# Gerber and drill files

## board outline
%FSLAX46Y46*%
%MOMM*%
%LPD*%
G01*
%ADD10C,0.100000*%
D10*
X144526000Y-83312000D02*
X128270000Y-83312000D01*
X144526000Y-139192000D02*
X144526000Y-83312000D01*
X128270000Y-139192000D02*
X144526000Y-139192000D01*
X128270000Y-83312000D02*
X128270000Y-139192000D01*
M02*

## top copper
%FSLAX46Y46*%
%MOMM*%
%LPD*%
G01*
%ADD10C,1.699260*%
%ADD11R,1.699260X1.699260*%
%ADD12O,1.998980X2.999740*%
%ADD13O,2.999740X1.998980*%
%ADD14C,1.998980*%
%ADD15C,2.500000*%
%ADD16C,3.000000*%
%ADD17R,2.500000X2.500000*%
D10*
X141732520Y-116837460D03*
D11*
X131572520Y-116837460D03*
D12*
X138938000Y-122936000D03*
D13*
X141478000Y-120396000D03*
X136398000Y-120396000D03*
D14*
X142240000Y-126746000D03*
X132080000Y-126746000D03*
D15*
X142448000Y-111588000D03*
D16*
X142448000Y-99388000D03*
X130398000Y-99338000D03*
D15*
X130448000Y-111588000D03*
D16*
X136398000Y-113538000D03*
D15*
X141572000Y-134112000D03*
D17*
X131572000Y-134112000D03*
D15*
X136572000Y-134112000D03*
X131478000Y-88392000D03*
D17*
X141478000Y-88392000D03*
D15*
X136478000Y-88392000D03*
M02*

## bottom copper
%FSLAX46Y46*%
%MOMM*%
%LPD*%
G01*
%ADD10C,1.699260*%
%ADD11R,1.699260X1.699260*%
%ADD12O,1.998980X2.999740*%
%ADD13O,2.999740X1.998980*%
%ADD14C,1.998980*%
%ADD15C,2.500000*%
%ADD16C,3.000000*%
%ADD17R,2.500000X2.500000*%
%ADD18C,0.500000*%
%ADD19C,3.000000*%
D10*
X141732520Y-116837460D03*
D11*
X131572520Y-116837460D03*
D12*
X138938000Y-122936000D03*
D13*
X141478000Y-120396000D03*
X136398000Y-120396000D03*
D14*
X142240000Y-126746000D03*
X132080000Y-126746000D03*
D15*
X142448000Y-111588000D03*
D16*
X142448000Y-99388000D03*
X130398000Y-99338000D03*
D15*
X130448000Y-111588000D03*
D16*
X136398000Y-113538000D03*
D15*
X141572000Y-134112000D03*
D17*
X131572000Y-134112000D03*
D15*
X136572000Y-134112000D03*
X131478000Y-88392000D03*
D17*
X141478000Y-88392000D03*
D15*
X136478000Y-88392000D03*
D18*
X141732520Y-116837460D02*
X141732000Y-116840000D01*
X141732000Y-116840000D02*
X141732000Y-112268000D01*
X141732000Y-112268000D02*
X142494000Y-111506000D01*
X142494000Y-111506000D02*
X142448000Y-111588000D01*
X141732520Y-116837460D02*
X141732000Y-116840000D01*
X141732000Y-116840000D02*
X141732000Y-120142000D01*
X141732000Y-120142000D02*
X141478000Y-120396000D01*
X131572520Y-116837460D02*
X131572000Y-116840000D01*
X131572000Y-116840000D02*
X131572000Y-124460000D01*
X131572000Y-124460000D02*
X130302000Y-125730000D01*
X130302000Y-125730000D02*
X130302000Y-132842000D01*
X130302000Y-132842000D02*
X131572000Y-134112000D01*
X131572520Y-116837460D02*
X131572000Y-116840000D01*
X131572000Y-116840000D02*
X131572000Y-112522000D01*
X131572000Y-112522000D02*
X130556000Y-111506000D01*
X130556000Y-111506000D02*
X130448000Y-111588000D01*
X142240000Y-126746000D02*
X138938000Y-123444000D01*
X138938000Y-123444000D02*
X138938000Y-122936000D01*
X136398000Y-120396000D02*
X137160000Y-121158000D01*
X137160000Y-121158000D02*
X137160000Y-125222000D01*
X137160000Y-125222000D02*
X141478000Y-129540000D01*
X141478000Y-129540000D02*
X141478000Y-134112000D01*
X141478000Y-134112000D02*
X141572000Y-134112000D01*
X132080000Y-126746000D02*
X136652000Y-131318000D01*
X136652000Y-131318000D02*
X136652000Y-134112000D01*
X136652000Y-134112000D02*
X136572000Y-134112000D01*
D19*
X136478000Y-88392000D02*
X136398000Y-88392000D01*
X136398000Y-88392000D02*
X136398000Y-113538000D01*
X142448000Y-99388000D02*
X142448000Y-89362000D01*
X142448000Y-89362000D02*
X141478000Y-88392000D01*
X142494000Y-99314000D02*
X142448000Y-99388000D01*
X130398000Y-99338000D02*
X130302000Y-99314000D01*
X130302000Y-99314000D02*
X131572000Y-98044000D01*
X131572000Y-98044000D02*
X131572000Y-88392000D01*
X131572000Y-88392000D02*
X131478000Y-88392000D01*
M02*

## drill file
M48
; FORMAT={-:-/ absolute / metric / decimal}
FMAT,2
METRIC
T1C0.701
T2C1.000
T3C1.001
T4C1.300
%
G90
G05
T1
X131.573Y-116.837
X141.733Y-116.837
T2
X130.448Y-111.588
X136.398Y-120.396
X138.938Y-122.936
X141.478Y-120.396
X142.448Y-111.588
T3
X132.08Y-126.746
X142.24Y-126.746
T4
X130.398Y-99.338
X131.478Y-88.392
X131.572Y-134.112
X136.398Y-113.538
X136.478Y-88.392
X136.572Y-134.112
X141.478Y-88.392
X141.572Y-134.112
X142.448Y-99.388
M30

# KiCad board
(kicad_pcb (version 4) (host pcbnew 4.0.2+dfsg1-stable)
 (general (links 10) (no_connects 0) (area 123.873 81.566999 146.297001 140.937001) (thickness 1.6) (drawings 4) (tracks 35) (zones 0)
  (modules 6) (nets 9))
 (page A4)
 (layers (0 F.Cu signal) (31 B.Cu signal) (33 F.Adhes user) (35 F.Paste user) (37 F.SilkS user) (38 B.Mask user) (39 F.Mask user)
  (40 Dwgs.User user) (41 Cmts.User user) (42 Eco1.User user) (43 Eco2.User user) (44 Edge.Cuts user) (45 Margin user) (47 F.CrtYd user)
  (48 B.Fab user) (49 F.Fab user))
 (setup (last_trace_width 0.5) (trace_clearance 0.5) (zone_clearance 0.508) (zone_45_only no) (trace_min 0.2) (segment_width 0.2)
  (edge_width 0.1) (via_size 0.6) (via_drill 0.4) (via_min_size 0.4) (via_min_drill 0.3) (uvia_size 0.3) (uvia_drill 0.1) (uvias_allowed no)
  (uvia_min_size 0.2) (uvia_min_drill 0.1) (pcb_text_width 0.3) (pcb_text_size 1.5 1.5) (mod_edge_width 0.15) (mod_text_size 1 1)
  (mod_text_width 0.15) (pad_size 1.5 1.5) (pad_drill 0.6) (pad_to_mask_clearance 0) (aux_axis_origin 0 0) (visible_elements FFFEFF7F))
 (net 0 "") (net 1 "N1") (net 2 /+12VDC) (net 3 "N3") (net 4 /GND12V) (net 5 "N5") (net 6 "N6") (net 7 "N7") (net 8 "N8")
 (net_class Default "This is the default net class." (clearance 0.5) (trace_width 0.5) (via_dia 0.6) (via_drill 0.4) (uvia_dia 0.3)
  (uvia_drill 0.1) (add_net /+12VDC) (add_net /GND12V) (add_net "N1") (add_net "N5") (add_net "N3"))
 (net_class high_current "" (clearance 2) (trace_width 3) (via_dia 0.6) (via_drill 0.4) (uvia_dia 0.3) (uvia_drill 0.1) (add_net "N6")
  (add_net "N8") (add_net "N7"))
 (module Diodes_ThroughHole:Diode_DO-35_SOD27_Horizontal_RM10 (layer F.Cu) (at 131.572 116.84)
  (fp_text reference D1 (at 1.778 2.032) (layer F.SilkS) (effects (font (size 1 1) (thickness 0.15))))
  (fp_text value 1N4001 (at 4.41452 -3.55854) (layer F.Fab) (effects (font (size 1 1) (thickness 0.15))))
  (pad 2 thru_hole circle (at 10.16052 -0.00254 180) (size 1.69926 1.69926) (drill 0.70104) (layers *.Cu *.Mask F.SilkS) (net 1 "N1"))
  (pad 1 thru_hole rect (at 0.00052 -0.00254 180) (size 1.69926 1.69926) (drill 0.70104) (layers *.Cu *.Mask F.SilkS) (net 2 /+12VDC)))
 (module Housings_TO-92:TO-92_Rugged (layer F.Cu) (at 141.478 120.396 180)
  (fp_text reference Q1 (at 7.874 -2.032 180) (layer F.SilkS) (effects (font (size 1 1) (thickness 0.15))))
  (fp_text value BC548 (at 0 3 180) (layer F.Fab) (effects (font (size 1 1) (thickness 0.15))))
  (pad 2 thru_hole oval (at 2.54 -2.54 270) (size 2.99974 1.99898) (drill 1) (layers *.Cu *.Mask F.SilkS) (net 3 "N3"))
  (pad 1 thru_hole oval (at 0 0 270) (size 1.99898 2.99974) (drill 1) (layers *.Cu *.Mask F.SilkS) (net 1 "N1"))
  (pad 3 thru_hole oval (at 5.08 0 270) (size 1.99898 2.99974) (drill 1) (layers *.Cu *.Mask F.SilkS) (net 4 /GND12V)))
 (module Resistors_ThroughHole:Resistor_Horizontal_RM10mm (layer F.Cu) (at 137.16 126.746 180)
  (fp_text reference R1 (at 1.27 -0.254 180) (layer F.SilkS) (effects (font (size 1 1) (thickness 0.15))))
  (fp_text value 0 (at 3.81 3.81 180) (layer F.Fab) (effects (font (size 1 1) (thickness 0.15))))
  (pad 1 thru_hole circle (at -5.08 0 180) (size 1.99898 1.99898) (drill 1.00076) (layers *.Cu *.SilkS *.Mask) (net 3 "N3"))
  (pad 2 thru_hole circle (at 5.08 0 180) (size 1.99898 1.99898) (drill 1.00076) (layers *.Cu *.SilkS *.Mask) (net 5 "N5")))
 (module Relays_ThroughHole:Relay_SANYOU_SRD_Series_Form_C (layer F.Cu) (at 136.398 113.538 90)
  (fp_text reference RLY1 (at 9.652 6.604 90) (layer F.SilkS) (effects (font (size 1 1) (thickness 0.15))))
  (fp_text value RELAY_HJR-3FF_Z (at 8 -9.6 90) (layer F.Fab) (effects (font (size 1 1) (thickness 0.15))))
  (pad 2 thru_hole circle (at 1.95 6.05 180) (size 2.5 2.5) (drill 1) (layers *.Cu *.Mask) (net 1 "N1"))
  (pad 3 thru_hole circle (at 14.15 6.05 180) (size 3 3) (drill 1.3) (layers *.Cu *.Mask) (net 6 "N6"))
  (pad 4 thru_hole circle (at 14.2 -6 180) (size 3 3) (drill 1.3) (layers *.Cu *.Mask) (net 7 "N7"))
  (pad 5 thru_hole circle (at 1.95 -5.95 180) (size 2.5 2.5) (drill 1) (layers *.Cu *.Mask F.SilkS) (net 2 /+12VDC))
  (pad 1 thru_hole circle (at 0 0 180) (size 3 3) (drill 1.3) (layers *.Cu *.Mask) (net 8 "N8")))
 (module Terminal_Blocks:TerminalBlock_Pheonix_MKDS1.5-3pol (layer F.Cu) (at 131.572 134.112)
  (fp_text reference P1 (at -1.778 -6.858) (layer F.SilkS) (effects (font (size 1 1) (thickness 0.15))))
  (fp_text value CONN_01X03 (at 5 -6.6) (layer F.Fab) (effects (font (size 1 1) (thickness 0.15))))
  (pad 3 thru_hole circle (at 10 0) (size 2.5 2.5) (drill 1.3) (layers *.Cu *.Mask F.SilkS) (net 4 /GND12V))
  (pad 1 thru_hole rect (at 0 0) (size 2.5 2.5) (drill 1.3) (layers *.Cu *.Mask F.SilkS) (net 2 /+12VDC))
  (pad 2 thru_hole circle (at 5 0) (size 2.5 2.5) (drill 1.3) (layers *.Cu *.Mask F.SilkS) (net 5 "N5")))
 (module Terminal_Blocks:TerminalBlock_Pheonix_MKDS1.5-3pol (layer F.Cu) (at 141.478 88.392 180)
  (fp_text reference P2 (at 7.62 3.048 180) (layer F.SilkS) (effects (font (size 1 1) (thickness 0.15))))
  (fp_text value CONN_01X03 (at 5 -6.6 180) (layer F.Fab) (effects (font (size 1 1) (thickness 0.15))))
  (pad 3 thru_hole circle (at 10 0 180) (size 2.5 2.5) (drill 1.3) (layers *.Cu *.Mask F.SilkS) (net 7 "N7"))
  (pad 1 thru_hole rect (at 0 0 180) (size 2.5 2.5) (drill 1.3) (layers *.Cu *.Mask F.SilkS) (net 6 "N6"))
  (pad 2 thru_hole circle (at 5 0 180) (size 2.5 2.5) (drill 1.3) (layers *.Cu *.Mask F.SilkS) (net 8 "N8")))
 (gr_line (start 144.526 83.312) (end 128.27 83.312) (angle 90) (layer Edge.Cuts) (width 0.1))
 (gr_line (start 144.526 139.192) (end 144.526 83.312) (angle 90) (layer Edge.Cuts) (width 0.1))
 (gr_line (start 128.27 139.192) (end 144.526 139.192) (angle 90) (layer Edge.Cuts) (width 0.1))
 (gr_line (start 128.27 83.312) (end 128.27 139.192) (angle 90) (layer Edge.Cuts) (width 0.1))
 (segment (start 141.73252 116.83746) (end 141.732 116.84) (width 0.5) (layer B.Cu) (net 1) (status 80000))
 (segment (start 141.732 116.84) (end 141.732 112.268) (width 0.5) (layer B.Cu) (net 1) (status 80000))
 (segment (start 141.732 112.268) (end 142.494 111.506) (width 0.5) (layer B.Cu) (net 1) (status 80000))
 (segment (start 142.494 111.506) (end 142.448 111.588) (width 0.5) (layer B.Cu) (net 1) (status 80000))
 (segment (start 141.73252 116.83746) (end 141.732 116.84) (width 0.5) (layer B.Cu) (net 1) (status 80000))
 (segment (start 141.732 116.84) (end 141.732 120.142) (width 0.5) (layer B.Cu) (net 1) (status 80000))
 (segment (start 141.732 120.142) (end 141.478 120.396) (width 0.5) (layer B.Cu) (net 1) (status 80000))
 (segment (start 131.57252 116.83746) (end 131.572 116.84) (width 0.5) (layer B.Cu) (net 2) (status 80000))
 (segment (start 131.572 116.84) (end 131.572 124.46) (width 0.5) (layer B.Cu) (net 2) (status 80000))
 (segment (start 131.572 124.46) (end 130.302 125.73) (width 0.5) (layer B.Cu) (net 2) (status 80000))
 (segment (start 130.302 125.73) (end 130.302 132.842) (width 0.5) (layer B.Cu) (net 2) (status 80000))
 (segment (start 130.302 132.842) (end 131.572 134.112) (width 0.5) (layer B.Cu) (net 2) (status 80000))
 (segment (start 131.57252 116.83746) (end 131.572 116.84) (width 0.5) (layer B.Cu) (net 2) (status 80000))
 (segment (start 131.572 116.84) (end 131.572 112.522) (width 0.5) (layer B.Cu) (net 2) (status 80000))
 (segment (start 131.572 112.522) (end 130.556 111.506) (width 0.5) (layer B.Cu) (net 2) (status 80000))
 (segment (start 130.556 111.506) (end 130.448 111.588) (width 0.5) (layer B.Cu) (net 2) (status 80000))
 (segment (start 142.24 126.746) (end 138.938 123.444) (width 0.5) (layer B.Cu) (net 3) (status 80000))
 (segment (start 138.938 123.444) (end 138.938 122.936) (width 0.5) (layer B.Cu) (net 3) (status 80000))
 (segment (start 136.398 120.396) (end 137.16 121.158) (width 0.5) (layer B.Cu) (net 4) (status 80000))
 (segment (start 137.16 121.158) (end 137.16 125.222) (width 0.5) (layer B.Cu) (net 4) (status 80000))
 (segment (start 137.16 125.222) (end 141.478 129.54) (width 0.5) (layer B.Cu) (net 4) (status 80000))
 (segment (start 141.478 129.54) (end 141.478 134.112) (width 0.5) (layer B.Cu) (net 4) (status 80000))
 (segment (start 141.478 134.112) (end 141.572 134.112) (width 0.5) (layer B.Cu) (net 4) (status 80000))
 (segment (start 132.08 126.746) (end 136.652 131.318) (width 0.5) (layer B.Cu) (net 5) (status 80000))
 (segment (start 136.652 131.318) (end 136.652 134.112) (width 0.5) (layer B.Cu) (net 5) (status 80000))
 (segment (start 136.652 134.112) (end 136.572 134.112) (width 0.5) (layer B.Cu) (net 5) (status 80000))
 (segment (start 136.478 88.392) (end 136.398 88.392) (width 3) (layer B.Cu) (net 8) (status 80000))
 (segment (start 136.398 88.392) (end 136.398 113.538) (width 3) (layer B.Cu) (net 8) (status 80000))
 (segment (start 142.448 99.388) (end 142.448 89.362) (width 3) (layer B.Cu) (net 6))
 (segment (start 142.448 89.362) (end 141.478 88.392) (width 3) (layer B.Cu) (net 6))
 (segment (start 142.494 99.314) (end 142.448 99.388) (width 3) (layer B.Cu) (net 6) (status 80000))
 (segment (start 130.398 99.338) (end 130.302 99.314) (width 3) (layer B.Cu) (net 7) (status 80000))
 (segment (start 130.302 99.314) (end 131.572 98.044) (width 3) (layer B.Cu) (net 7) (status 80000))
 (segment (start 131.572 98.044) (end 131.572 88.392) (width 3) (layer B.Cu) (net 7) (status 80000))
 (segment (start 131.572 88.392) (end 131.478 88.392) (width 3) (layer B.Cu) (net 7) (status 80000)))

